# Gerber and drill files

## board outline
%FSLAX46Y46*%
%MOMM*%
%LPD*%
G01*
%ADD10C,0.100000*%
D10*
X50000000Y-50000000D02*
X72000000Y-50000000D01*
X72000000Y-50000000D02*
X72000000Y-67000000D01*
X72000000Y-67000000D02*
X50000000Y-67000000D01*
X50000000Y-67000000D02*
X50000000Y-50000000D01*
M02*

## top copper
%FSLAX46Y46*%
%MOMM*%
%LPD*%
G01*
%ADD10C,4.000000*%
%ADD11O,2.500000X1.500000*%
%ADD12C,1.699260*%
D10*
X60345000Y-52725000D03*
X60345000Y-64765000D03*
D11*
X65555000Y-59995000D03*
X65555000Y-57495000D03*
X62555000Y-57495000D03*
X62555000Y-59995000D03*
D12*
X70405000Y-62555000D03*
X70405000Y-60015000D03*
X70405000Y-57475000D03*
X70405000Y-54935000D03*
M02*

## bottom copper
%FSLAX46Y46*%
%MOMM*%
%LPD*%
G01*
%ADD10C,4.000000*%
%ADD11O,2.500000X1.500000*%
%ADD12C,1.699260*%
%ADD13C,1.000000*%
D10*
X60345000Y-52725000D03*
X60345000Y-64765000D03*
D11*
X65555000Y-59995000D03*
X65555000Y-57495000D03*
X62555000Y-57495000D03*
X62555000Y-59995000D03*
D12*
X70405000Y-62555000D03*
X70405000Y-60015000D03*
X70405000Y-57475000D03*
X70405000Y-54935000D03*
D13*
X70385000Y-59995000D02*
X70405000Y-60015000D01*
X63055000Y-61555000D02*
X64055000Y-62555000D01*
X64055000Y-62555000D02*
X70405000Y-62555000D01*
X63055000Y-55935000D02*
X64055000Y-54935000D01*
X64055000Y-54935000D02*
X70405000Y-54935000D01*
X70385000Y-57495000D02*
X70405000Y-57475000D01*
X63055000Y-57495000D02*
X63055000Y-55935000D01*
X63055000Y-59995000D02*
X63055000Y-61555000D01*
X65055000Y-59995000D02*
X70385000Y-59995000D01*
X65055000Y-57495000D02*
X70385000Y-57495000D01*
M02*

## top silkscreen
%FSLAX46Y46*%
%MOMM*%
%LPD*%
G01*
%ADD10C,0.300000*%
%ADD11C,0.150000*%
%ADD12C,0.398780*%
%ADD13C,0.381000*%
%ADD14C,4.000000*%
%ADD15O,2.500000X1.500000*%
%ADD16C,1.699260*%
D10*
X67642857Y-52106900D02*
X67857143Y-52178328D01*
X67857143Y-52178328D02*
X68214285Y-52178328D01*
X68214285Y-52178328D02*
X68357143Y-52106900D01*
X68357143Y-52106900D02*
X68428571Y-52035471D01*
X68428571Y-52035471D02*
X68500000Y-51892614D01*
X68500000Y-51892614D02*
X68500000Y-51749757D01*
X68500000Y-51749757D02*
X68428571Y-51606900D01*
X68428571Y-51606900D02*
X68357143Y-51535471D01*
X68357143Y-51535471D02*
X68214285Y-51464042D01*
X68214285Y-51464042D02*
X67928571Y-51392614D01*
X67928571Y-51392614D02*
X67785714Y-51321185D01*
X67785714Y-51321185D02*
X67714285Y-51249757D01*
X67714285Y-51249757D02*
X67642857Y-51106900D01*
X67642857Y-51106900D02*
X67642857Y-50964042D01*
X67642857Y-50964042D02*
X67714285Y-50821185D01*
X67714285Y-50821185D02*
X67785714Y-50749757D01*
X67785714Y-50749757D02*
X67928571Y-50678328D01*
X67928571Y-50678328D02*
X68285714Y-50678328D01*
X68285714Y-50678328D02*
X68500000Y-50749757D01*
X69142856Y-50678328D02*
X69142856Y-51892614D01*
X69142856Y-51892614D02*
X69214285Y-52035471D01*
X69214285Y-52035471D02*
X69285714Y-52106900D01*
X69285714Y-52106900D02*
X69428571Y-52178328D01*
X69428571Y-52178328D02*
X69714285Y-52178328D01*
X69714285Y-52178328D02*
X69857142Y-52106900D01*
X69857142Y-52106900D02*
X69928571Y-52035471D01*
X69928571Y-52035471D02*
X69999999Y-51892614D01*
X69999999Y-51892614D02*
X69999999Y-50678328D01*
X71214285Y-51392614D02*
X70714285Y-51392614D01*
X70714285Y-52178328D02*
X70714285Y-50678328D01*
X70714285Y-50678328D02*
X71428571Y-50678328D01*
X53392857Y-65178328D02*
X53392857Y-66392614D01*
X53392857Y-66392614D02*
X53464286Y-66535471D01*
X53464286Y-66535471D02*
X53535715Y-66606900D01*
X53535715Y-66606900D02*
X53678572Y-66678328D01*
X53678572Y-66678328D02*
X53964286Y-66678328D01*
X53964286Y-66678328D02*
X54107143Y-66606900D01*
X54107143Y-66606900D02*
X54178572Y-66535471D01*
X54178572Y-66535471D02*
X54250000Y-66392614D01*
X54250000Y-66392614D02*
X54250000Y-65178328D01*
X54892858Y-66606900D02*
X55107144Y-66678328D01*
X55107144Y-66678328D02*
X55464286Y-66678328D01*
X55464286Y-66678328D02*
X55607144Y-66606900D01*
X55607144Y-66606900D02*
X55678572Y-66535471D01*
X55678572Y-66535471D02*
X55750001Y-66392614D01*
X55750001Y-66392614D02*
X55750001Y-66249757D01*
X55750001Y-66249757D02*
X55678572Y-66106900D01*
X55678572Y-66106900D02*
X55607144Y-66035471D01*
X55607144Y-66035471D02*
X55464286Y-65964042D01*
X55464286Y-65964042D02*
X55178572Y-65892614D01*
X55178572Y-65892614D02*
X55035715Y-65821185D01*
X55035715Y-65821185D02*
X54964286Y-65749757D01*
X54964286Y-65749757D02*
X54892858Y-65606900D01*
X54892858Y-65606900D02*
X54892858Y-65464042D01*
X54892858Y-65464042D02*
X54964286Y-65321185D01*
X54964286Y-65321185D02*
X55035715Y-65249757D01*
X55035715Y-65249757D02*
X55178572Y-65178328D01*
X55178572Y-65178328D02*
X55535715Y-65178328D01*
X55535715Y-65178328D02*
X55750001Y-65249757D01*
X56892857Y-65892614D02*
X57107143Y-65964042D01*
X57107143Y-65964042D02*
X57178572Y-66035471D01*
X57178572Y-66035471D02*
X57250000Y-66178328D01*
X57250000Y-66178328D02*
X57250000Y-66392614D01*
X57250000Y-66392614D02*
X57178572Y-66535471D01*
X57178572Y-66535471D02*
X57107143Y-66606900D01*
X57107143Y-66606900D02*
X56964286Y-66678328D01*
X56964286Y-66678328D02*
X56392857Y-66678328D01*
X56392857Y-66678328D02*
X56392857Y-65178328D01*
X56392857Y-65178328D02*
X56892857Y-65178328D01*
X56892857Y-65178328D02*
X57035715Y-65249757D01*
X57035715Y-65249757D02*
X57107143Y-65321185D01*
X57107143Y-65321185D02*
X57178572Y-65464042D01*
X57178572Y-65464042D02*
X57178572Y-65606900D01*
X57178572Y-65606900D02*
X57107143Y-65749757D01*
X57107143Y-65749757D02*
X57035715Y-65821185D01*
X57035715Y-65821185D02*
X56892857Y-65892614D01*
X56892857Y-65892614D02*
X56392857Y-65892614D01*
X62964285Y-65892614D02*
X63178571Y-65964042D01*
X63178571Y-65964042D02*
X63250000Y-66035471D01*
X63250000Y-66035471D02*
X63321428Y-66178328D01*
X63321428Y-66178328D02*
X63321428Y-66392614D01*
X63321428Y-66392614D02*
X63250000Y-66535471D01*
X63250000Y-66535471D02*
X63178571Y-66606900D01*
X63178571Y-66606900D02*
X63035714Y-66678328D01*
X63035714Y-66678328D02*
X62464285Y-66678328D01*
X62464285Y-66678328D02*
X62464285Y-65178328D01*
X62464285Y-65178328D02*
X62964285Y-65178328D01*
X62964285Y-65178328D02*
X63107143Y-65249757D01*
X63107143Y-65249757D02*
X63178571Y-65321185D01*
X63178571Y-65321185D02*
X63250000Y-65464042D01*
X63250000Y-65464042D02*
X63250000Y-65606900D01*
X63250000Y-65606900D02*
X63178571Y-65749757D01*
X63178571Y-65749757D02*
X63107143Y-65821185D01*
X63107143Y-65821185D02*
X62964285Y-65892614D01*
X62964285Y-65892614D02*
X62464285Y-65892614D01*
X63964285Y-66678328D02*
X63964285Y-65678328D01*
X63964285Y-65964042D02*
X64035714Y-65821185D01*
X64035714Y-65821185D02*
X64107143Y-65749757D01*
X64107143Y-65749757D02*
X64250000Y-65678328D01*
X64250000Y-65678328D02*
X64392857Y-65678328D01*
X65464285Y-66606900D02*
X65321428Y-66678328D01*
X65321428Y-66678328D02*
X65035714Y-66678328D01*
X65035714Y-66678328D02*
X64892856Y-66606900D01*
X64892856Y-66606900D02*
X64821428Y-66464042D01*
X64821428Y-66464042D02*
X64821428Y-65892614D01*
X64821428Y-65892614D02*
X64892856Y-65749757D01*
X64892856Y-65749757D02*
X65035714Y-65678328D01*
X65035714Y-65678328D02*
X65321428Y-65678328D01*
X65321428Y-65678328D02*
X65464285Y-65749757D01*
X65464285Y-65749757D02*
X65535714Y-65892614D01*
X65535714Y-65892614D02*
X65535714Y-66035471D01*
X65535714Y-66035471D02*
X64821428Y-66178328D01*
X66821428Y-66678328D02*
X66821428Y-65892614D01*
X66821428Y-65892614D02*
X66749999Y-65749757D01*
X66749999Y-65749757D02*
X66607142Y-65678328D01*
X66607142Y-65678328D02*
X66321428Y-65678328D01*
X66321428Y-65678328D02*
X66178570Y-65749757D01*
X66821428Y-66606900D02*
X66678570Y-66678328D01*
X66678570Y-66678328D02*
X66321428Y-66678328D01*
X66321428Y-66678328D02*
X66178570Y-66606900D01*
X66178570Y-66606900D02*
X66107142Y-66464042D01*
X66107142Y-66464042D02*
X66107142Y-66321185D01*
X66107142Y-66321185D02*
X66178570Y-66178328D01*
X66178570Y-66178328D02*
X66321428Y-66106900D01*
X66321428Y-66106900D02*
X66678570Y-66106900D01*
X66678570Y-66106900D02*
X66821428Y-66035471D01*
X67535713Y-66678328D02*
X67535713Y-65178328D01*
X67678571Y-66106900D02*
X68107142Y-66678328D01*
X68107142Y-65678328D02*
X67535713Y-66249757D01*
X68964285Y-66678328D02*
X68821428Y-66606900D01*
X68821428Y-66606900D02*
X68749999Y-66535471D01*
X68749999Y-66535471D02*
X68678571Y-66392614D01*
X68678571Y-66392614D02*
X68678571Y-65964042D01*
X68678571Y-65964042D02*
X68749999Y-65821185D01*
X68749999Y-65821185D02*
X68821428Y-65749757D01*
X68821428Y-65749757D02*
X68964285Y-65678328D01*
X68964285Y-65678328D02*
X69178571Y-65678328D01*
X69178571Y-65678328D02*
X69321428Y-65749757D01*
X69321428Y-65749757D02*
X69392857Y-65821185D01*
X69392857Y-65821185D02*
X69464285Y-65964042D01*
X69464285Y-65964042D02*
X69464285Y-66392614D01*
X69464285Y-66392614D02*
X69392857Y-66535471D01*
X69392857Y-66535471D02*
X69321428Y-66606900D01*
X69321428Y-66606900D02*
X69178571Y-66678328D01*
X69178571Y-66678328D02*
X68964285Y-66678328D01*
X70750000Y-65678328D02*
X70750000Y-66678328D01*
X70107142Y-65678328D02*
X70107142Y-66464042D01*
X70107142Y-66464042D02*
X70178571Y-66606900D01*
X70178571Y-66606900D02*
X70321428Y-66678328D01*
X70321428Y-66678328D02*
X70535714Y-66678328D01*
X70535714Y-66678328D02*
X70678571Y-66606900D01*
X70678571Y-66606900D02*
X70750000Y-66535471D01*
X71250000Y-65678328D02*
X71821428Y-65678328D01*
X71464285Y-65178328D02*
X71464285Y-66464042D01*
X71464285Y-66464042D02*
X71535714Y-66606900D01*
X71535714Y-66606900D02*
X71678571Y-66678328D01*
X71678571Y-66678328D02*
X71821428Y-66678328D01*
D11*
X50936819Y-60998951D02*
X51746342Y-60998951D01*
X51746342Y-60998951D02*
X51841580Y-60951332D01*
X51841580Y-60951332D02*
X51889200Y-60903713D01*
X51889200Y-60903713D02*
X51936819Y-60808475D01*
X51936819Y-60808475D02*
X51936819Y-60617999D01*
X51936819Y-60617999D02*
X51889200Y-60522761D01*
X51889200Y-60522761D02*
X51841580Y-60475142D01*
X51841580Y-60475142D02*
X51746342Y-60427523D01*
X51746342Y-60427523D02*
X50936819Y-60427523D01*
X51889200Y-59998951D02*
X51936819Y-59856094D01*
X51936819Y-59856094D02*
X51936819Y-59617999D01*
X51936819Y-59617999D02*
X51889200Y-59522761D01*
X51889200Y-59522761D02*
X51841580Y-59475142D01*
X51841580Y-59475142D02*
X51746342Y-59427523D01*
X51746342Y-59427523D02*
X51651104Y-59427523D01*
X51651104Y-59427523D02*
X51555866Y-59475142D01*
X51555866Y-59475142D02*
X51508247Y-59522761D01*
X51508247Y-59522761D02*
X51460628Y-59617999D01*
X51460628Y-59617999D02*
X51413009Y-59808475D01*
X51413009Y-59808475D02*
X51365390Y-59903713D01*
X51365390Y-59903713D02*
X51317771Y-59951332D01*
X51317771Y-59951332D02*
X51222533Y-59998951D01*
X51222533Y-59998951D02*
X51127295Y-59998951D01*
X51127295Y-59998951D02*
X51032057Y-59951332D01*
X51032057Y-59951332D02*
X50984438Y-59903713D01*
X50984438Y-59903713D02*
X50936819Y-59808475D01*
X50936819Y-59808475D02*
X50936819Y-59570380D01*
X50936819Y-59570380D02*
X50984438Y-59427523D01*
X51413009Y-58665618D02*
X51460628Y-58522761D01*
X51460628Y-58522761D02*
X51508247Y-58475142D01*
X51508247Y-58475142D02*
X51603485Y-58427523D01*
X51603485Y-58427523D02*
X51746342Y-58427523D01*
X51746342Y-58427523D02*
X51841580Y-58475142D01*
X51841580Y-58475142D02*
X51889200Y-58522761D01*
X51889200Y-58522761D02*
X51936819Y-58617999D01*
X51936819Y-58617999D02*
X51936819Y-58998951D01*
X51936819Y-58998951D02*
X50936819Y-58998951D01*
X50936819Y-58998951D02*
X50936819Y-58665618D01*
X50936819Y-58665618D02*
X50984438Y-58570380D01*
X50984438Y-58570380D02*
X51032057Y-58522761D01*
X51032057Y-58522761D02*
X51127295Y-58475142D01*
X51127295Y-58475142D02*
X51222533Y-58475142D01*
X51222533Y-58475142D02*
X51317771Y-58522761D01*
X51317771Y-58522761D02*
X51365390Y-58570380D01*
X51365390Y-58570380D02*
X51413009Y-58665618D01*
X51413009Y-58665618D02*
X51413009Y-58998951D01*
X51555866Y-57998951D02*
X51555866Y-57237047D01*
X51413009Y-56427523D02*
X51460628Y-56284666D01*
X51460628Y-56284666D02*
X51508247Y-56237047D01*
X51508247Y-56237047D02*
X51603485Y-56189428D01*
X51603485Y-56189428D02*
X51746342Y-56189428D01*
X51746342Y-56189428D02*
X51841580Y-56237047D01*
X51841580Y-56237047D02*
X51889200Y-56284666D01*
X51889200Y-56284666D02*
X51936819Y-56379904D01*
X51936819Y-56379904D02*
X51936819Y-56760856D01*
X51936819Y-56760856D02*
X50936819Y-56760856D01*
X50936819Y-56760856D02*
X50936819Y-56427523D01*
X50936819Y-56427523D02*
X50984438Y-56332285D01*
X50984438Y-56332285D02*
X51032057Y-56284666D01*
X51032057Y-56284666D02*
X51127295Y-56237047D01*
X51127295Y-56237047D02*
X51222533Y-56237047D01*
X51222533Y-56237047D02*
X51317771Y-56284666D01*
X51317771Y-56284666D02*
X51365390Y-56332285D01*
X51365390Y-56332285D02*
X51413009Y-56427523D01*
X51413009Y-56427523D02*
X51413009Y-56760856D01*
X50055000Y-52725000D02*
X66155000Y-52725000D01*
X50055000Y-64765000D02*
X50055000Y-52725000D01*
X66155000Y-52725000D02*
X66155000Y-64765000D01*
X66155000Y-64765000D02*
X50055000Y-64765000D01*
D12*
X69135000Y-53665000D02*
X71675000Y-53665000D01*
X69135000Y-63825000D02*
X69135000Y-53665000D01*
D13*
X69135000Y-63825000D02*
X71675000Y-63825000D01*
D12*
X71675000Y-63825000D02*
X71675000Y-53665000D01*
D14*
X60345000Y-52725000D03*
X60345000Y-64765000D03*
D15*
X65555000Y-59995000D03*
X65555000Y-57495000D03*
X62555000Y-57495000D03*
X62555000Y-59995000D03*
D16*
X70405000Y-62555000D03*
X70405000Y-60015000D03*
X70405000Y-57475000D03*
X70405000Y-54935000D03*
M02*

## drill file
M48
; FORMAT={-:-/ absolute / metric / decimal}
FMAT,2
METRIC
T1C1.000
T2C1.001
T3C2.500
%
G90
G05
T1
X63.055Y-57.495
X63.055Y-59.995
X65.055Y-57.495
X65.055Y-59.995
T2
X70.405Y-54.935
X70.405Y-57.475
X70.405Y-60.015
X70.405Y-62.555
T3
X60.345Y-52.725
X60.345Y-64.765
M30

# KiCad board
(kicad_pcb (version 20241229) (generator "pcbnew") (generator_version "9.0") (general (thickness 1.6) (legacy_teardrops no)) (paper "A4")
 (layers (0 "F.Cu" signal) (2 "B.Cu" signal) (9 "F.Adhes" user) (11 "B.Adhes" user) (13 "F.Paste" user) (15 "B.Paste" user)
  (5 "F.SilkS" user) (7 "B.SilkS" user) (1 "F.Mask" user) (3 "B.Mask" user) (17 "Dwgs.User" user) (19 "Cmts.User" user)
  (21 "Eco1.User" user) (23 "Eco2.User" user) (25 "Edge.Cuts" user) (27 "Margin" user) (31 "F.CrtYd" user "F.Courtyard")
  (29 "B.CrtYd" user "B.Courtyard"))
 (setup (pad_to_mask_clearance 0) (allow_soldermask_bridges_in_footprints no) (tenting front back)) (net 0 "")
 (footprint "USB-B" (layer "F.Cu") (at 64.055 58.745 -90)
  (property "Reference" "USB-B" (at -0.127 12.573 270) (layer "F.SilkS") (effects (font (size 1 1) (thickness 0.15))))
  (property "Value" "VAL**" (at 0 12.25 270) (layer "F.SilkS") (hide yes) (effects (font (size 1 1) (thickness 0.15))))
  (fp_line (start -6.02 14) (end -6.02 -2.1) (stroke (width 0.15) (type solid)) (layer "F.SilkS"))
  (fp_line (start 6.02 14) (end -6.02 14) (stroke (width 0.15) (type solid)) (layer "F.SilkS"))
  (fp_line (start -6.02 -2.1) (end 6.02 -2.1) (stroke (width 0.15) (type solid)) (layer "F.SilkS"))
  (fp_line (start 6.02 -2.1) (end 6.02 14) (stroke (width 0.15) (type solid)) (layer "F.SilkS"))
  (pad "" thru_hole circle (at -6.02 3.71 270) (size 4 4) (drill 2.5) (layers "*.Cu" "*.Mask" "F.SilkS") (remove_unused_layers no))
  (pad "" thru_hole circle (at 6.02 3.71 270) (size 4 4) (drill 2.5) (layers "*.Cu" "*.Mask" "F.SilkS") (remove_unused_layers no))
  (pad "1" thru_hole oval (at 1.25 -1 270) (size 1.5 2.5) (drill 1 (offset 0 -0.5)) (layers "*.Cu" "*.Mask" "F.SilkS")
   (remove_unused_layers no))
  (pad "2" thru_hole oval (at -1.25 -1 270) (size 1.5 2.5) (drill 1 (offset 0 -0.5)) (layers "*.Cu" "*.Mask" "F.SilkS")
   (remove_unused_layers no))
  (pad "3" thru_hole oval (at -1.25 1 270) (size 1.5 2.5) (drill 1 (offset 0 0.5)) (layers "*.Cu" "*.Mask" "F.SilkS")
   (remove_unused_layers no))
  (pad "4" thru_hole oval (at 1.25 1 270) (size 1.5 2.5) (drill 1 (offset 0 0.5)) (layers "*.Cu" "*.Mask" "F.SilkS")
   (remove_unused_layers no)))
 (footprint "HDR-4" (layer "F.Cu") (at 70.405 58.745 90)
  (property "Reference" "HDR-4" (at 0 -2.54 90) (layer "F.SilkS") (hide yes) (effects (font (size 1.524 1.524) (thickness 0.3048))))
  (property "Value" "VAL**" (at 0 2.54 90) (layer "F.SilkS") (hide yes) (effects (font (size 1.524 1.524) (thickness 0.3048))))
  (fp_line (start 5.08 -1.27) (end 5.08 1.27) (stroke (width 0.39878) (type solid)) (layer "F.SilkS"))
  (fp_line (start -5.08 -1.27) (end 5.08 -1.27) (stroke (width 0.39878) (type solid)) (layer "F.SilkS"))
  (fp_line (start -5.08 -1.27) (end -5.08 1.27) (stroke (width 0.381) (type solid)) (layer "F.SilkS"))
  (fp_line (start -5.08 1.27) (end 5.08 1.27) (stroke (width 0.39878) (type solid)) (layer "F.SilkS"))
  (pad "1" thru_hole circle (at -3.81 0 90) (size 1.69926 1.69926) (drill 1.00076) (layers "*.Cu" "*.Mask" "F.SilkS")
   (remove_unused_layers no))
  (pad "2" thru_hole circle (at -1.27 0 90) (size 1.69926 1.69926) (drill 1.00076) (layers "*.Cu" "*.Mask" "F.SilkS")
   (remove_unused_layers no))
  (pad "3" thru_hole circle (at 1.27 0 90) (size 1.69926 1.69926) (drill 1.00076) (layers "*.Cu" "*.Mask" "F.SilkS")
   (remove_unused_layers no))
  (pad "4" thru_hole circle (at 3.81 0 90) (size 1.69926 1.69926) (drill 1.00076) (layers "*.Cu" "*.Mask" "F.SilkS")
   (remove_unused_layers no)))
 (gr_line (start 50 50) (end 72 50) (stroke (width 0.1) (type solid)) (layer "Edge.Cuts"))
 (gr_line (start 72 50) (end 72 67) (stroke (width 0.1) (type solid)) (layer "Edge.Cuts"))
 (gr_line (start 72 67) (end 50 67) (stroke (width 0.1) (type solid)) (layer "Edge.Cuts"))
 (gr_line (start 50 67) (end 50 50) (stroke (width 0.1) (type solid)) (layer "Edge.Cuts"))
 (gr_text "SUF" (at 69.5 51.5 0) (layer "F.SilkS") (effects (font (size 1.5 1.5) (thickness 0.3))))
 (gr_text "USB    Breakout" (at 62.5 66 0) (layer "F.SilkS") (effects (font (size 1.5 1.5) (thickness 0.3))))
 (segment (start 70.385 59.995) (end 70.405 60.015) (width 1) (layer "B.Cu") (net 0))
 (segment (start 63.055 61.555) (end 64.055 62.555) (width 1) (layer "B.Cu") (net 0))
 (segment (start 64.055 62.555) (end 70.405 62.555) (width 1) (layer "B.Cu") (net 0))
 (segment (start 63.055 55.935) (end 64.055 54.935) (width 1) (layer "B.Cu") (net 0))
 (segment (start 64.055 54.935) (end 70.405 54.935) (width 1) (layer "B.Cu") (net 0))
 (segment (start 70.385 57.495) (end 70.405 57.475) (width 1) (layer "B.Cu") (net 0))
 (segment (start 63.055 57.495) (end 63.055 55.935) (width 1) (layer "B.Cu") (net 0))
 (segment (start 63.055 59.995) (end 63.055 61.555) (width 1) (layer "B.Cu") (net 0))
 (segment (start 65.055 59.995) (end 70.385 59.995) (width 1) (layer "B.Cu") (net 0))
 (segment (start 65.055 57.495) (end 70.385 57.495) (width 1) (layer "B.Cu") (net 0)))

